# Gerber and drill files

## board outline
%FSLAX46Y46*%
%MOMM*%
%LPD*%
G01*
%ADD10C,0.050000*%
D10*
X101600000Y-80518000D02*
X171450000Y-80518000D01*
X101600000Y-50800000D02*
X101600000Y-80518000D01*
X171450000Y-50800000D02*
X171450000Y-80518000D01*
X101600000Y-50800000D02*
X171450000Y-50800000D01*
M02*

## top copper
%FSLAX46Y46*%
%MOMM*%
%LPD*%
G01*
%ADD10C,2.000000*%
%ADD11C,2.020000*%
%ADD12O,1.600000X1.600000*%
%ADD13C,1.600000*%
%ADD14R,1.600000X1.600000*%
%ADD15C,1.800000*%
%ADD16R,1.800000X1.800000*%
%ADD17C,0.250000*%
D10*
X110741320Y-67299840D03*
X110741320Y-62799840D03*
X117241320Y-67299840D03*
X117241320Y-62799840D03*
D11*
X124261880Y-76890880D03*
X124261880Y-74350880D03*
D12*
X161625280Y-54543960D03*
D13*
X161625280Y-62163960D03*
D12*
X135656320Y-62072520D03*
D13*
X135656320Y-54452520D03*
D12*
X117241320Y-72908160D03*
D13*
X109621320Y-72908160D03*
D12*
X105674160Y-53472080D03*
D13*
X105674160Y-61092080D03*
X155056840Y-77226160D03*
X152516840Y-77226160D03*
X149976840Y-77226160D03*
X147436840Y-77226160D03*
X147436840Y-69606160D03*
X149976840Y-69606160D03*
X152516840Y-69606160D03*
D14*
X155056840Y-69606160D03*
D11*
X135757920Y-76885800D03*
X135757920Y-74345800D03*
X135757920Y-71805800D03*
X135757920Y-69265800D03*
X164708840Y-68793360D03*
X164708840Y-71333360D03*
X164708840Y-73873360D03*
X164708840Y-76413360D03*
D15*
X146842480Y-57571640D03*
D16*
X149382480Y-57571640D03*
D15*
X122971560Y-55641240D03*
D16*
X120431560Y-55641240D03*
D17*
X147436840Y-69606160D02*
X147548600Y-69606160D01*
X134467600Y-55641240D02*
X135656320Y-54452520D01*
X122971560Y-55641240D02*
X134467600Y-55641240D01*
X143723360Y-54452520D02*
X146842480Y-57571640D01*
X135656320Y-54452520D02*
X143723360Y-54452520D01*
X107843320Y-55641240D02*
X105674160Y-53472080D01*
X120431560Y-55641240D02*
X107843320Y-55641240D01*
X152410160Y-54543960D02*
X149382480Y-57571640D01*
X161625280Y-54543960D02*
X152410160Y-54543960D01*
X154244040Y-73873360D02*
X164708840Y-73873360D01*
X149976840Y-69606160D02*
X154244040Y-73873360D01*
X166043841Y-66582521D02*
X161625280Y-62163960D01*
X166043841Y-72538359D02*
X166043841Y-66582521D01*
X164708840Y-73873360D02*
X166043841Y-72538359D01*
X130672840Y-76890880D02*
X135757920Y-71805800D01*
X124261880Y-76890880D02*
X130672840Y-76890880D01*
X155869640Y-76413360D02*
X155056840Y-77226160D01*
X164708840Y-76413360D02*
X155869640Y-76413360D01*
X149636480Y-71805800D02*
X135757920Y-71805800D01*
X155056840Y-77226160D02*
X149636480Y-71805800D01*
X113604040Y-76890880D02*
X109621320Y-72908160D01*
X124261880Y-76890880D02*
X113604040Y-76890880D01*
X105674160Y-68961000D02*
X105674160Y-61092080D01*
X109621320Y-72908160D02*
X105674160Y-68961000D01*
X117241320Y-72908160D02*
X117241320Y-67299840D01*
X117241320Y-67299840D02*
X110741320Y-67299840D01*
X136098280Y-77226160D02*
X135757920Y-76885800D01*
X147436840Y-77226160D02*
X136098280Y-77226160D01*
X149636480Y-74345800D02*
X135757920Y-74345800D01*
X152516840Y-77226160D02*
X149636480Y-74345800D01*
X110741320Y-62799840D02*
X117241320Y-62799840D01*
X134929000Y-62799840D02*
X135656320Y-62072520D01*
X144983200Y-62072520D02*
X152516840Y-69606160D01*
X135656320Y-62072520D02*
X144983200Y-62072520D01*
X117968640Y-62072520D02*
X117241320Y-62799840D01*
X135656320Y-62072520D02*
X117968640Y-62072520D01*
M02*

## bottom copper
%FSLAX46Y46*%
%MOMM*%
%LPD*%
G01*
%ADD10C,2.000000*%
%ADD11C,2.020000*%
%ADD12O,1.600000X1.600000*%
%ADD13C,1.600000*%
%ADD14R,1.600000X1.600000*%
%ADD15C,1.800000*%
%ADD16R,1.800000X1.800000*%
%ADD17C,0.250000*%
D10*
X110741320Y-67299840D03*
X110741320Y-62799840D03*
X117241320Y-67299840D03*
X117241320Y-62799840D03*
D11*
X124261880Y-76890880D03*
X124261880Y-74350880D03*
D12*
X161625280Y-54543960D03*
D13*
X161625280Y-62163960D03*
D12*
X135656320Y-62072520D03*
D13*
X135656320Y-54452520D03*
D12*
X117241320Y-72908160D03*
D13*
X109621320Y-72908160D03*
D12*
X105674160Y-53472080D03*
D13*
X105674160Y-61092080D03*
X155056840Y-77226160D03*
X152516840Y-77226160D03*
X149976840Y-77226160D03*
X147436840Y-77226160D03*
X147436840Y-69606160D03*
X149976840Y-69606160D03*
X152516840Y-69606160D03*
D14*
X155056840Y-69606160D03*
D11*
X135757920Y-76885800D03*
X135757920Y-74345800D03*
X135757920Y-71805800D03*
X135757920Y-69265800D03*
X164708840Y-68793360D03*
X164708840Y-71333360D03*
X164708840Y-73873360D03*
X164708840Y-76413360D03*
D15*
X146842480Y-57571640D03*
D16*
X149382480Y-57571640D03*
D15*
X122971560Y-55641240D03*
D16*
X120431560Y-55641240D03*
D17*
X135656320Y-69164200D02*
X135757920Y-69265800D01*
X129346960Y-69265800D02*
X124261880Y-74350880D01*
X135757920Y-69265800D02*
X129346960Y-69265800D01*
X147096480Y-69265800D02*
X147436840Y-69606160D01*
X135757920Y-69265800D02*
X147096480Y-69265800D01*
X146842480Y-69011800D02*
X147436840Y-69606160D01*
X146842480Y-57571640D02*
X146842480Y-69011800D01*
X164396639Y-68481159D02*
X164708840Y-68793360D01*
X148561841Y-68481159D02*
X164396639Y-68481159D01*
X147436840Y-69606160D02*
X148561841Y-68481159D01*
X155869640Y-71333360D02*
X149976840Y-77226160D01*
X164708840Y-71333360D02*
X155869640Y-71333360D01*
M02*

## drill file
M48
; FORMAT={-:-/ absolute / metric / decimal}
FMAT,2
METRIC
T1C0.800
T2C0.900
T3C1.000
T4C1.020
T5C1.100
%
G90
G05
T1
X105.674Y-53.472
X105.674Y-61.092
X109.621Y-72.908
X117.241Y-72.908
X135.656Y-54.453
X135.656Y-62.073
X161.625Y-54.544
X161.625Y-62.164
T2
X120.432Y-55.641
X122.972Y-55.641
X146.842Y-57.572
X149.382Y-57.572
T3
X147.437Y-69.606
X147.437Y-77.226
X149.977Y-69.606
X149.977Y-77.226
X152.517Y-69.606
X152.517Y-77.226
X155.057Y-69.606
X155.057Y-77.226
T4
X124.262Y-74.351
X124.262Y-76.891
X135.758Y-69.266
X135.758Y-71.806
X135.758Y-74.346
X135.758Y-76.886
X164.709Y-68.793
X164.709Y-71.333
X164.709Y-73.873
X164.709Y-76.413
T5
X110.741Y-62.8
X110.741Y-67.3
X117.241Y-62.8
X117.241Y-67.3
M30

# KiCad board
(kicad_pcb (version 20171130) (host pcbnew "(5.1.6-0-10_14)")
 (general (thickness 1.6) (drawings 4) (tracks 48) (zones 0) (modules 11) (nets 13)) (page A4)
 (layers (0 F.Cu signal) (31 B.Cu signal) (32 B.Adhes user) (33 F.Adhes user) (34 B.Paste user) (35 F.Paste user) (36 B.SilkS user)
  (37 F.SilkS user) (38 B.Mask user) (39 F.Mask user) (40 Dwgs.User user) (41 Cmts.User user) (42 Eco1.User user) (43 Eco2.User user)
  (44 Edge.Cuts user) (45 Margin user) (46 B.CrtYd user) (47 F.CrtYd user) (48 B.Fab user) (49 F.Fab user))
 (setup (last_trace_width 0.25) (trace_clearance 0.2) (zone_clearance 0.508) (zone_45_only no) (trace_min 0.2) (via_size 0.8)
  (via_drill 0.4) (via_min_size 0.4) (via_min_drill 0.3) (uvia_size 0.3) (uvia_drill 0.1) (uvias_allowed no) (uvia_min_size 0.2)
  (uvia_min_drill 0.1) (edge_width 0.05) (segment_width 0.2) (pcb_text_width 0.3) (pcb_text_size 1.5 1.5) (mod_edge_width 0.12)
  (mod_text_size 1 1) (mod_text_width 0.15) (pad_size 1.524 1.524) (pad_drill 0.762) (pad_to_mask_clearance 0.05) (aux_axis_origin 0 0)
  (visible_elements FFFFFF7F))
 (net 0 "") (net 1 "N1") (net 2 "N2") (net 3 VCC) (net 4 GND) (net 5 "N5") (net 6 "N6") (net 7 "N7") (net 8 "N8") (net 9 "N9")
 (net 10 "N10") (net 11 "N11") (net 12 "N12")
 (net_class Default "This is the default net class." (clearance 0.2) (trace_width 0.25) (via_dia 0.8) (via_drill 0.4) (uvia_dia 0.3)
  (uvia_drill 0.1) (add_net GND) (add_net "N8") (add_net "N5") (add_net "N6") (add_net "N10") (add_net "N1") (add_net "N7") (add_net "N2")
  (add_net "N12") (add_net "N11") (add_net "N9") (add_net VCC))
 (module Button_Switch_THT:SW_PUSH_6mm (layer F.Cu) (at 117.24132 67.29984 180)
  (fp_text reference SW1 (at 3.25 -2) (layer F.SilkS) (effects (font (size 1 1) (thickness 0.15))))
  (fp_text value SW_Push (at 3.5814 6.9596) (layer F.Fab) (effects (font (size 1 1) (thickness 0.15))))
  (pad 1 thru_hole circle (at 6.5 0 270) (size 2 2) (drill 1.1) (layers *.Cu *.Mask) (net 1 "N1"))
  (pad 2 thru_hole circle (at 6.5 4.5 270) (size 2 2) (drill 1.1) (layers *.Cu *.Mask) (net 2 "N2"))
  (pad 1 thru_hole circle (at 0 0 270) (size 2 2) (drill 1.1) (layers *.Cu *.Mask) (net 1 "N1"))
  (pad 2 thru_hole circle (at 0 4.5 270) (size 2 2) (drill 1.1) (layers *.Cu *.Mask) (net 2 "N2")))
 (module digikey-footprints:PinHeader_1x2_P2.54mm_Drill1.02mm (layer F.Cu) (at 124.26188 74.35088 270)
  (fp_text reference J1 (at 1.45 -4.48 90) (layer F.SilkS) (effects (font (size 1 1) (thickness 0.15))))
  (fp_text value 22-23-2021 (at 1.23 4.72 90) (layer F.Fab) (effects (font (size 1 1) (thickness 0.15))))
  (pad 2 thru_hole circle (at 2.54 0 270) (size 2.02 2.02) (drill 1.02) (layers *.Cu *.Mask) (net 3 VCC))
  (pad 1 thru_hole circle (at 0 0 270) (size 2.02 2.02) (drill 1.02) (layers *.Cu *.Mask) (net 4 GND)))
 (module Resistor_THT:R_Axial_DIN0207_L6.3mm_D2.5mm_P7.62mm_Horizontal (layer F.Cu) (at 161.62528 62.16396 90)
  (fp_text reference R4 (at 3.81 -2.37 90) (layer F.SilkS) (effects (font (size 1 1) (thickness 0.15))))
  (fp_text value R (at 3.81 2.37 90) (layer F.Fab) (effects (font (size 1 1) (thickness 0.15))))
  (pad 2 thru_hole oval (at 7.62 0 90) (size 1.6 1.6) (drill 0.8) (layers *.Cu *.Mask) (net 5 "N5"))
  (pad 1 thru_hole circle (at 0 0 90) (size 1.6 1.6) (drill 0.8) (layers *.Cu *.Mask) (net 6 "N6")))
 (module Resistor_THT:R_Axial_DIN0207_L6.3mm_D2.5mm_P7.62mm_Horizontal (layer F.Cu) (at 135.65632 54.45252 270)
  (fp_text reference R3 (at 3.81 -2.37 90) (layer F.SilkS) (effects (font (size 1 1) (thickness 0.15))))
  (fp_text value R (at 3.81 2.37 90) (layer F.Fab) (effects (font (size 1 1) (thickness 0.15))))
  (pad 2 thru_hole oval (at 7.62 0 270) (size 1.6 1.6) (drill 0.8) (layers *.Cu *.Mask) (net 2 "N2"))
  (pad 1 thru_hole circle (at 0 0 270) (size 1.6 1.6) (drill 0.8) (layers *.Cu *.Mask) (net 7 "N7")))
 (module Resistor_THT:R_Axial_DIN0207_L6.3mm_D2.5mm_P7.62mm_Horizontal (layer F.Cu) (at 109.62132 72.90816)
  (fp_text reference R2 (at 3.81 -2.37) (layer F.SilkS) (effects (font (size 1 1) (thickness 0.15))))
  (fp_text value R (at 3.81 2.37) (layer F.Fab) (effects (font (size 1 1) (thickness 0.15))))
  (pad 2 thru_hole oval (at 7.62 0) (size 1.6 1.6) (drill 0.8) (layers *.Cu *.Mask) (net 1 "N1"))
  (pad 1 thru_hole circle (at 0 0) (size 1.6 1.6) (drill 0.8) (layers *.Cu *.Mask) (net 3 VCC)))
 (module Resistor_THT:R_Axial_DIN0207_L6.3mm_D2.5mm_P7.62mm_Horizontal (layer F.Cu) (at 105.67416 61.09208 90)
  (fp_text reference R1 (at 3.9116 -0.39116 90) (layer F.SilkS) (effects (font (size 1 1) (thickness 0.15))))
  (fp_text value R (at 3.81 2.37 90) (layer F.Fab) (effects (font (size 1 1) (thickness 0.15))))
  (pad 2 thru_hole oval (at 7.62 0 90) (size 1.6 1.6) (drill 0.8) (layers *.Cu *.Mask) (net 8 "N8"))
  (pad 1 thru_hole circle (at 0 0 90) (size 1.6 1.6) (drill 0.8) (layers *.Cu *.Mask) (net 3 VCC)))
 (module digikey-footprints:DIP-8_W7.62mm (layer F.Cu) (at 155.05684 69.60616 270)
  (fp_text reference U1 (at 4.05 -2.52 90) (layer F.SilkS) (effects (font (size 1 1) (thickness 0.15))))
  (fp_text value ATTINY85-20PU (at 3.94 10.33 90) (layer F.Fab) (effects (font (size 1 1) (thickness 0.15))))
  (pad 8 thru_hole circle (at 7.62 0 270) (size 1.6 1.6) (drill 1) (layers *.Cu *.Mask) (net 3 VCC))
  (pad 7 thru_hole circle (at 7.62 2.54 270) (size 1.6 1.6) (drill 1) (layers *.Cu *.Mask) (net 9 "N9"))
  (pad 6 thru_hole circle (at 7.62 5.08 270) (size 1.6 1.6) (drill 1) (layers *.Cu *.Mask) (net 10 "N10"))
  (pad 5 thru_hole circle (at 7.62 7.62 270) (size 1.6 1.6) (drill 1) (layers *.Cu *.Mask) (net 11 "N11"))
  (pad 4 thru_hole circle (at 0 7.62 270) (size 1.6 1.6) (drill 1) (layers *.Cu *.Mask) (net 4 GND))
  (pad 3 thru_hole circle (at 0 5.08 270) (size 1.6 1.6) (drill 1) (layers *.Cu *.Mask) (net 6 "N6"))
  (pad 2 thru_hole circle (at 0 2.54 270) (size 1.6 1.6) (drill 1) (layers *.Cu *.Mask) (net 2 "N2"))
  (pad 1 thru_hole rect (at 0 0 270) (size 1.6 1.6) (drill 1) (layers *.Cu *.Mask) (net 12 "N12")))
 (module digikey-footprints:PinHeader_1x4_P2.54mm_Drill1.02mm (layer F.Cu) (at 135.75792 69.2658 270)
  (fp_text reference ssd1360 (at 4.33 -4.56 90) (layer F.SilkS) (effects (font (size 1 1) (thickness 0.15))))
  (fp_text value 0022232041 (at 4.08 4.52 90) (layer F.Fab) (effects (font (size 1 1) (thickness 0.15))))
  (pad 4 thru_hole circle (at 7.62 0 270) (size 2.02 2.02) (drill 1.02) (layers *.Cu *.Mask) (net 11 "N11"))
  (pad 3 thru_hole circle (at 5.08 0 270) (size 2.02 2.02) (drill 1.02) (layers *.Cu *.Mask) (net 9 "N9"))
  (pad 2 thru_hole circle (at 2.54 0 270) (size 2.02 2.02) (drill 1.02) (layers *.Cu *.Mask) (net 3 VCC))
  (pad 1 thru_hole circle (at 0 0 270) (size 2.02 2.02) (drill 1.02) (layers *.Cu *.Mask) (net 4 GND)))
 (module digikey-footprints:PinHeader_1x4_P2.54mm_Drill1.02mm (layer F.Cu) (at 164.70884 76.41336 90)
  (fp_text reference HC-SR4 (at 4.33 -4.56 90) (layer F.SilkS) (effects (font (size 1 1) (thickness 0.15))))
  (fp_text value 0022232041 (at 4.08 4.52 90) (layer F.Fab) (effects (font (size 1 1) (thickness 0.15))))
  (pad 4 thru_hole circle (at 7.62 0 90) (size 2.02 2.02) (drill 1.02) (layers *.Cu *.Mask) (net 4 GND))
  (pad 3 thru_hole circle (at 5.08 0 90) (size 2.02 2.02) (drill 1.02) (layers *.Cu *.Mask) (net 10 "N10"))
  (pad 2 thru_hole circle (at 2.54 0 90) (size 2.02 2.02) (drill 1.02) (layers *.Cu *.Mask) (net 6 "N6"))
  (pad 1 thru_hole circle (at 0 0 90) (size 2.02 2.02) (drill 1.02) (layers *.Cu *.Mask) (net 3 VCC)))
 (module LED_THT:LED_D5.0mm (layer F.Cu) (at 149.38248 57.57164 180)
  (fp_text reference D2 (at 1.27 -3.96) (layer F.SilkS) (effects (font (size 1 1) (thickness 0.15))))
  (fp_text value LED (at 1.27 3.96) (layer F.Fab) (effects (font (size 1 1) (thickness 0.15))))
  (pad 2 thru_hole circle (at 2.54 0 180) (size 1.8 1.8) (drill 0.9) (layers *.Cu *.Mask) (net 4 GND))
  (pad 1 thru_hole rect (at 0 0 180) (size 1.8 1.8) (drill 0.9) (layers *.Cu *.Mask) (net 5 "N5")))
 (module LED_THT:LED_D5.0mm (layer F.Cu) (at 120.43156 55.64124)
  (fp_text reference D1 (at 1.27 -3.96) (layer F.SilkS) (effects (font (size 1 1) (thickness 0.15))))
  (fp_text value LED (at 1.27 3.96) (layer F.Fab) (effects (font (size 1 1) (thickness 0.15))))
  (pad 2 thru_hole circle (at 2.54 0) (size 1.8 1.8) (drill 0.9) (layers *.Cu *.Mask) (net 4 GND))
  (pad 1 thru_hole rect (at 0 0) (size 1.8 1.8) (drill 0.9) (layers *.Cu *.Mask) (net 8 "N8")))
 (gr_line (start 101.6 80.518) (end 171.45 80.518) (layer Edge.Cuts) (width 0.05))
 (gr_line (start 101.6 50.8) (end 101.6 80.518) (layer Edge.Cuts) (width 0.05))
 (gr_line (start 171.45 50.8) (end 171.45 80.518) (layer Edge.Cuts) (width 0.05))
 (gr_line (start 101.6 50.8) (end 171.45 50.8) (layer Edge.Cuts) (width 0.05))
 (segment (start 147.43684 69.60616) (end 147.5486 69.60616) (width 0.25) (layer F.Cu) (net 4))
 (segment (start 135.65632 69.1642) (end 135.75792 69.2658) (width 0.25) (layer B.Cu) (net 4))
 (segment (start 129.34696 69.2658) (end 124.26188 74.35088) (width 0.25) (layer B.Cu) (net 4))
 (segment (start 135.75792 69.2658) (end 129.34696 69.2658) (width 0.25) (layer B.Cu) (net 4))
 (segment (start 147.09648 69.2658) (end 147.43684 69.60616) (width 0.25) (layer B.Cu) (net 4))
 (segment (start 135.75792 69.2658) (end 147.09648 69.2658) (width 0.25) (layer B.Cu) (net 4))
 (segment (start 134.4676 55.64124) (end 135.65632 54.45252) (width 0.25) (layer F.Cu) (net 4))
 (segment (start 122.97156 55.64124) (end 134.4676 55.64124) (width 0.25) (layer F.Cu) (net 4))
 (segment (start 143.72336 54.45252) (end 146.84248 57.57164) (width 0.25) (layer F.Cu) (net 4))
 (segment (start 135.65632 54.45252) (end 143.72336 54.45252) (width 0.25) (layer F.Cu) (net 4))
 (segment (start 146.84248 69.0118) (end 147.43684 69.60616) (width 0.25) (layer B.Cu) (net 4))
 (segment (start 146.84248 57.57164) (end 146.84248 69.0118) (width 0.25) (layer B.Cu) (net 4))
 (segment (start 164.396639 68.481159) (end 164.70884 68.79336) (width 0.25) (layer B.Cu) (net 4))
 (segment (start 148.561841 68.481159) (end 164.396639 68.481159) (width 0.25) (layer B.Cu) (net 4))
 (segment (start 147.43684 69.60616) (end 148.561841 68.481159) (width 0.25) (layer B.Cu) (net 4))
 (segment (start 107.84332 55.64124) (end 105.67416 53.47208) (width 0.25) (layer F.Cu) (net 8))
 (segment (start 120.43156 55.64124) (end 107.84332 55.64124) (width 0.25) (layer F.Cu) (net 8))
 (segment (start 152.41016 54.54396) (end 149.38248 57.57164) (width 0.25) (layer F.Cu) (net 5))
 (segment (start 161.62528 54.54396) (end 152.41016 54.54396) (width 0.25) (layer F.Cu) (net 5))
 (segment (start 155.86964 71.33336) (end 149.97684 77.22616) (width 0.25) (layer B.Cu) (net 10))
 (segment (start 164.70884 71.33336) (end 155.86964 71.33336) (width 0.25) (layer B.Cu) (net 10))
 (segment (start 154.24404 73.87336) (end 164.70884 73.87336) (width 0.25) (layer F.Cu) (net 6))
 (segment (start 149.97684 69.60616) (end 154.24404 73.87336) (width 0.25) (layer F.Cu) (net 6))
 (segment (start 166.043841 66.582521) (end 161.62528 62.16396) (width 0.25) (layer F.Cu) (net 6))
 (segment (start 166.043841 72.538359) (end 166.043841 66.582521) (width 0.25) (layer F.Cu) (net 6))
 (segment (start 164.70884 73.87336) (end 166.043841 72.538359) (width 0.25) (layer F.Cu) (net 6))
 (segment (start 130.67284 76.89088) (end 135.75792 71.8058) (width 0.25) (layer F.Cu) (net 3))
 (segment (start 124.26188 76.89088) (end 130.67284 76.89088) (width 0.25) (layer F.Cu) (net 3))
 (segment (start 155.86964 76.41336) (end 155.05684 77.22616) (width 0.25) (layer F.Cu) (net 3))
 (segment (start 164.70884 76.41336) (end 155.86964 76.41336) (width 0.25) (layer F.Cu) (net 3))
 (segment (start 149.63648 71.8058) (end 135.75792 71.8058) (width 0.25) (layer F.Cu) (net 3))
 (segment (start 155.05684 77.22616) (end 149.63648 71.8058) (width 0.25) (layer F.Cu) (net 3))
 (segment (start 113.60404 76.89088) (end 109.62132 72.90816) (width 0.25) (layer F.Cu) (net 3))
 (segment (start 124.26188 76.89088) (end 113.60404 76.89088) (width 0.25) (layer F.Cu) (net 3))
 (segment (start 105.67416 68.961) (end 105.67416 61.09208) (width 0.25) (layer F.Cu) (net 3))
 (segment (start 109.62132 72.90816) (end 105.67416 68.961) (width 0.25) (layer F.Cu) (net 3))
 (segment (start 117.24132 72.90816) (end 117.24132 67.29984) (width 0.25) (layer F.Cu) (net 1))
 (segment (start 117.24132 67.29984) (end 110.74132 67.29984) (width 0.25) (layer F.Cu) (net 1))
 (segment (start 136.09828 77.22616) (end 135.75792 76.8858) (width 0.25) (layer F.Cu) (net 11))
 (segment (start 147.43684 77.22616) (end 136.09828 77.22616) (width 0.25) (layer F.Cu) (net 11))
 (segment (start 149.63648 74.3458) (end 135.75792 74.3458) (width 0.25) (layer F.Cu) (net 9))
 (segment (start 152.51684 77.22616) (end 149.63648 74.3458) (width 0.25) (layer F.Cu) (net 9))
 (segment (start 110.74132 62.79984) (end 117.24132 62.79984) (width 0.25) (layer F.Cu) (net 2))
 (segment (start 134.929 62.79984) (end 135.65632 62.07252) (width 0.25) (layer F.Cu) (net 2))
 (segment (start 144.9832 62.07252) (end 152.51684 69.60616) (width 0.25) (layer F.Cu) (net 2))
 (segment (start 135.65632 62.07252) (end 144.9832 62.07252) (width 0.25) (layer F.Cu) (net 2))
 (segment (start 117.96864 62.07252) (end 117.24132 62.79984) (width 0.25) (layer F.Cu) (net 2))
 (segment (start 135.65632 62.07252) (end 117.96864 62.07252) (width 0.25) (layer F.Cu) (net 2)))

